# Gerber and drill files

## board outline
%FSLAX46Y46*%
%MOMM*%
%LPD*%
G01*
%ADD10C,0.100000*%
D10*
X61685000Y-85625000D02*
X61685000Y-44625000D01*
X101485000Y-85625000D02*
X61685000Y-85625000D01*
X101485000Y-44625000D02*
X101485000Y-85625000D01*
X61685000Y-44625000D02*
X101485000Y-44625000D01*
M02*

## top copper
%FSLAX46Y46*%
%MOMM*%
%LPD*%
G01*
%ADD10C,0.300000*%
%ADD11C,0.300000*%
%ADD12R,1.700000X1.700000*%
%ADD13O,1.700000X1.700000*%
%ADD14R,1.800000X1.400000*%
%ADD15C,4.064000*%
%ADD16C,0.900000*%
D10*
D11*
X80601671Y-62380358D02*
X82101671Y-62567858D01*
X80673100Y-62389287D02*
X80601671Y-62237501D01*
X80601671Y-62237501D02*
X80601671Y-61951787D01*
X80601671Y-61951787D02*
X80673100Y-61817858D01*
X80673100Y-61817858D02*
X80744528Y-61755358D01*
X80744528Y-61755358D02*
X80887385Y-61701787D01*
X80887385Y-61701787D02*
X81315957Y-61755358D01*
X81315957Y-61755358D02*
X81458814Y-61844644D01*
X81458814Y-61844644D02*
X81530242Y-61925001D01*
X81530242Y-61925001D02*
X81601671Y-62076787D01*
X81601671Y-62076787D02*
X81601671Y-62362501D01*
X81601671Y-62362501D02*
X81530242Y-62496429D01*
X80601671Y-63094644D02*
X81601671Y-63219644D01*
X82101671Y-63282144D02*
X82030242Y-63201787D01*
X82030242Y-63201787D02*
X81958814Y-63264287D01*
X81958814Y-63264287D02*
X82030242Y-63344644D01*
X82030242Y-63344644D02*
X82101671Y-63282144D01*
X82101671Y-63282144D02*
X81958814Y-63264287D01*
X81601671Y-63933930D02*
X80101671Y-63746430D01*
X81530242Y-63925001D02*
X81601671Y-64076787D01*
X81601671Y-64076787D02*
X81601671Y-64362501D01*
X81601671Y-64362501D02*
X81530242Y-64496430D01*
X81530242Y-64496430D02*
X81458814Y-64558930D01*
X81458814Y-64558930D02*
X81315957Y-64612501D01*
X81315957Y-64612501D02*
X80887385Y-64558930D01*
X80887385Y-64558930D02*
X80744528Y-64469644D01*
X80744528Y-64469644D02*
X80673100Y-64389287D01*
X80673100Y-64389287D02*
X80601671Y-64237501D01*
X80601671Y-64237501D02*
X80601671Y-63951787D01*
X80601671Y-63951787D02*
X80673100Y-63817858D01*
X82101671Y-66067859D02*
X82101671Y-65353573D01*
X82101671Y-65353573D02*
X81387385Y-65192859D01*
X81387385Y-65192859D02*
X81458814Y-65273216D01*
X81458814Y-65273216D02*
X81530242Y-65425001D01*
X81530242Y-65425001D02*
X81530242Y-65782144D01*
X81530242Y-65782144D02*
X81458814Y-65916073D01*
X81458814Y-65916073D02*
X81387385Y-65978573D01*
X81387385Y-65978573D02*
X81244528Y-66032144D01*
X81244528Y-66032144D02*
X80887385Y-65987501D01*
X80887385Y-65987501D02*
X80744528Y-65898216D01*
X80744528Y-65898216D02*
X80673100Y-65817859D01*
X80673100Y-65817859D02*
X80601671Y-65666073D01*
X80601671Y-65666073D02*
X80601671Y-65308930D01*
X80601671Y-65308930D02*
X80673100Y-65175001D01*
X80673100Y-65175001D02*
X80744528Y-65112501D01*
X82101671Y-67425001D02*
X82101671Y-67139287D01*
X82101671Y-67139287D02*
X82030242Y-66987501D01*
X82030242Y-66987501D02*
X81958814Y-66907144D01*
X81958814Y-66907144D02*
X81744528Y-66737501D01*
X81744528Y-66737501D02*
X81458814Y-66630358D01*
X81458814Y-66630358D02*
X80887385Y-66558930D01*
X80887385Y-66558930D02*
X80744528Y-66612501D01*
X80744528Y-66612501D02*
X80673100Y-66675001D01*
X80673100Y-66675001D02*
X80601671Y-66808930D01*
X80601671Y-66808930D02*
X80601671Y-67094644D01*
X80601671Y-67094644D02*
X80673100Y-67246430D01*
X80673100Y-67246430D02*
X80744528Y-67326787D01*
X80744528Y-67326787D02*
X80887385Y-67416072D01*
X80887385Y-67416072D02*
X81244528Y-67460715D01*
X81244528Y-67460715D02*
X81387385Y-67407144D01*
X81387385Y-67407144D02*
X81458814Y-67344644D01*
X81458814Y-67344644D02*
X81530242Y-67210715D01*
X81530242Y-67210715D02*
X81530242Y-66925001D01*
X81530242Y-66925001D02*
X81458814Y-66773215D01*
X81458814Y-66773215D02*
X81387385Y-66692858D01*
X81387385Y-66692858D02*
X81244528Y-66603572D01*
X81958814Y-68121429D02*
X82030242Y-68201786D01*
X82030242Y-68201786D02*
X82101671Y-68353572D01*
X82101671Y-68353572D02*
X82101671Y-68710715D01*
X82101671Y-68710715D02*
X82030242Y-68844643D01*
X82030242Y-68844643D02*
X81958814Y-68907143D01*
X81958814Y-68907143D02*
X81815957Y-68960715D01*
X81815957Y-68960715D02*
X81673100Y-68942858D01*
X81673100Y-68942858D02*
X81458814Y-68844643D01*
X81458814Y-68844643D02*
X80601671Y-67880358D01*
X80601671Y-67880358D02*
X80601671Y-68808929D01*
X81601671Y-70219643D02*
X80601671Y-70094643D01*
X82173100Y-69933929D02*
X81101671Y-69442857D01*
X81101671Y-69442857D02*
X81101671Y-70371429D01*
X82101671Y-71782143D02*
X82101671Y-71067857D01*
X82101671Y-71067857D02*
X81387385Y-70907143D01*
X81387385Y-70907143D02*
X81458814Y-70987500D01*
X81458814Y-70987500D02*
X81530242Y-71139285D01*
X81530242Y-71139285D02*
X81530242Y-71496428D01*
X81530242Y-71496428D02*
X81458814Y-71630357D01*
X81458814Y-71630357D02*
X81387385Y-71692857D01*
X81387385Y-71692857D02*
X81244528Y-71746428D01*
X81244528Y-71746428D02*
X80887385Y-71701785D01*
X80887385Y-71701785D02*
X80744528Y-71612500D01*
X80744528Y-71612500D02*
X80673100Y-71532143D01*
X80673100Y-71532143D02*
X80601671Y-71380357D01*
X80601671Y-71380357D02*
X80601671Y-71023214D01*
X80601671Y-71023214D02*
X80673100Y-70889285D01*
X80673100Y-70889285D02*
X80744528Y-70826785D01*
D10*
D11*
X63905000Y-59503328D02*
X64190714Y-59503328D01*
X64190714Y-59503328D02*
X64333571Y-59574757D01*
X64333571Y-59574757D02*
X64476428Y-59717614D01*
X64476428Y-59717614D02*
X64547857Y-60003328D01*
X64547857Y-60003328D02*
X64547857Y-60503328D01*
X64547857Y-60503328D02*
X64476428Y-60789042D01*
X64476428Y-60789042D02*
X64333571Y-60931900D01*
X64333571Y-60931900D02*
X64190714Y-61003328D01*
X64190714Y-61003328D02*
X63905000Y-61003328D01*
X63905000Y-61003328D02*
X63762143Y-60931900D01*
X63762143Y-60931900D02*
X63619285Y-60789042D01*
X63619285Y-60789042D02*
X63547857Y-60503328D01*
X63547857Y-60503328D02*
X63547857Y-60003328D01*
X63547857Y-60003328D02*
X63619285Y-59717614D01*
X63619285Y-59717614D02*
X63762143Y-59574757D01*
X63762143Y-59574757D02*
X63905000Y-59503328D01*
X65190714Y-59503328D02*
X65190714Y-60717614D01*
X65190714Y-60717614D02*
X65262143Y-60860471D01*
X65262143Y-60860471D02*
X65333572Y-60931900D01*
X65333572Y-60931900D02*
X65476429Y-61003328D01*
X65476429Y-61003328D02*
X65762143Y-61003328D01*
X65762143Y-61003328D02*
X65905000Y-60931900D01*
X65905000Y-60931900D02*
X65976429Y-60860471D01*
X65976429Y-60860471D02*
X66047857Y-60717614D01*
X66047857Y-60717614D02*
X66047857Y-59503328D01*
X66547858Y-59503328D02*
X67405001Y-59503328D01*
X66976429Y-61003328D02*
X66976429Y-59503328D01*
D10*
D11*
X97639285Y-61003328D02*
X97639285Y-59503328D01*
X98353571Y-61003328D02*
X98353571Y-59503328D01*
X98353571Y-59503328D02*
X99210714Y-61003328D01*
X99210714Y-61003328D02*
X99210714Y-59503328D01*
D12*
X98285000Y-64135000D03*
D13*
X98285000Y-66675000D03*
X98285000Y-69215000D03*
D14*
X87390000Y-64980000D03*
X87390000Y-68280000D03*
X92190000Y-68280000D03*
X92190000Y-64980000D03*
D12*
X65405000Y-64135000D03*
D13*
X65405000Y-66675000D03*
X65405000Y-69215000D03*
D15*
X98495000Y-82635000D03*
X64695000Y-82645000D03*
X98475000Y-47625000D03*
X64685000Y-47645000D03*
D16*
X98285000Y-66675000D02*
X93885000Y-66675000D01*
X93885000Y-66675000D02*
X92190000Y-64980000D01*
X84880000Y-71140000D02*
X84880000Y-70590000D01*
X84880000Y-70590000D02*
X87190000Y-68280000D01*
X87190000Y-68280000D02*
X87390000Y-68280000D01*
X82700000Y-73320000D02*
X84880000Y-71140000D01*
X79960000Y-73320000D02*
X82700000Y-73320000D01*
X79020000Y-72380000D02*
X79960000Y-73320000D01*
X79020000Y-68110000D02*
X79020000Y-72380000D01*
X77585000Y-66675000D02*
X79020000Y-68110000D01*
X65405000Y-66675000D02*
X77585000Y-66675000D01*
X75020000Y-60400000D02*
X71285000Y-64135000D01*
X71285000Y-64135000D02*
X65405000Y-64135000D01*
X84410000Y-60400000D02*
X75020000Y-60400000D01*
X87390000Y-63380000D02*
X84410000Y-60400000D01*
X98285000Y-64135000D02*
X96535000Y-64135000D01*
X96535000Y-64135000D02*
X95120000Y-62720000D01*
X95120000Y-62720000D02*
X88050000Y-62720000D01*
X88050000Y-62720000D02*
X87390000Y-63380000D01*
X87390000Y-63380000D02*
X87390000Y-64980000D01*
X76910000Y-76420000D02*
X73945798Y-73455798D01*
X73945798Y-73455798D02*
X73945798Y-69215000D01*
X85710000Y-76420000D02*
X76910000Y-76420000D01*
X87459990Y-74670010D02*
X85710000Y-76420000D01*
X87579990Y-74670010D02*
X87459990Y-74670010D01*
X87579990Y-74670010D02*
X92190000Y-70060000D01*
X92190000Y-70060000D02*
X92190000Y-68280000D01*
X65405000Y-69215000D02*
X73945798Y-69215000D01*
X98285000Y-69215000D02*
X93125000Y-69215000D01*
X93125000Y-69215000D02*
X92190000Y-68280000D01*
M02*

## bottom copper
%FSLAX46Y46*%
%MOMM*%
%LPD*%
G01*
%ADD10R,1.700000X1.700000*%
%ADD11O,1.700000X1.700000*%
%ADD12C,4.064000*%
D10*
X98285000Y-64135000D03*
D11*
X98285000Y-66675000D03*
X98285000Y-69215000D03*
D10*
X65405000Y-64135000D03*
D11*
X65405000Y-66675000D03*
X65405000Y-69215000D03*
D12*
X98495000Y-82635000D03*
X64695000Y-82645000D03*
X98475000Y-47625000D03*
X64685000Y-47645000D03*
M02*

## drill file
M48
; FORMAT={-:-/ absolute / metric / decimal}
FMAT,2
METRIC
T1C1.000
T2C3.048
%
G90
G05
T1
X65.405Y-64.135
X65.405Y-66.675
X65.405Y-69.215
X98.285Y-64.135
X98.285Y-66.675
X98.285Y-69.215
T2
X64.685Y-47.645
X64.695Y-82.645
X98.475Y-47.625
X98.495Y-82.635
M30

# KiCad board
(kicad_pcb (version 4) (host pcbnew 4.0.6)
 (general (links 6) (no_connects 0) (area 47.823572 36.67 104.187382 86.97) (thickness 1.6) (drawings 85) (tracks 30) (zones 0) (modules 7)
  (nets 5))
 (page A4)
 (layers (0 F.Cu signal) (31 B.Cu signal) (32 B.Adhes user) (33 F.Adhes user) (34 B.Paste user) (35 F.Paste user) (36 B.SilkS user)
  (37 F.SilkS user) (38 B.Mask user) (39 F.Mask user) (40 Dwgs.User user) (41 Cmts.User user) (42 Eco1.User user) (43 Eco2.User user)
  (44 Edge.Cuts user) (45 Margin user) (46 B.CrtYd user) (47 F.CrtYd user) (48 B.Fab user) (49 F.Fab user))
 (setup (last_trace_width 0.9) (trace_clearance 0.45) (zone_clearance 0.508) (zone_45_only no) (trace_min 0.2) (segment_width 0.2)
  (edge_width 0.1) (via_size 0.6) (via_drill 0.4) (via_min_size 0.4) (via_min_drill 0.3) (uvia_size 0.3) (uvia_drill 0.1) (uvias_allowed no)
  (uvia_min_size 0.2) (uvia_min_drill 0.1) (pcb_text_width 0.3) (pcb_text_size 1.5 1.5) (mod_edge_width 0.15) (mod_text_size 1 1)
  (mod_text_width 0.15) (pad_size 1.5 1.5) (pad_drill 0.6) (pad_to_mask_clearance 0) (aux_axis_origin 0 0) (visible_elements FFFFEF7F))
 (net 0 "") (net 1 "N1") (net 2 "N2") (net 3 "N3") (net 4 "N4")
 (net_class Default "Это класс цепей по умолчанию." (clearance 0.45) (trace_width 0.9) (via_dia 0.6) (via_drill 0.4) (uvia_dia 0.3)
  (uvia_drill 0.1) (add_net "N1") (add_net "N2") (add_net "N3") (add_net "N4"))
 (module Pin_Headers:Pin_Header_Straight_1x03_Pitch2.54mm (layer F.Cu) (at 98.285 64.135)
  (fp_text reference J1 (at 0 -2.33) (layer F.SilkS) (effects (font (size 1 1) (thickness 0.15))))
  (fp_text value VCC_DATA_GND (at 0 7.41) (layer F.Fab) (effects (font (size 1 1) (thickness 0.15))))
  (pad 1 thru_hole rect (at 0 0) (size 1.7 1.7) (drill 1) (layers *.Cu *.Mask) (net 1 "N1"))
  (pad 2 thru_hole oval (at 0 2.54) (size 1.7 1.7) (drill 1) (layers *.Cu *.Mask) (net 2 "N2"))
  (pad 3 thru_hole oval (at 0 5.08) (size 1.7 1.7) (drill 1) (layers *.Cu *.Mask) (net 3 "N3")))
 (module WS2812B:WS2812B (layer F.Cu) (at 89.79 66.63 90)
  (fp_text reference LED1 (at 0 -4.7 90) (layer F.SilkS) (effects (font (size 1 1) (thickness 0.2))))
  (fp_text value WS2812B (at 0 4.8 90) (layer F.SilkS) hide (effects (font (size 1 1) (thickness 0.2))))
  (pad 1 smd rect (at 1.65 -2.4 90) (size 1.4 1.8) (layers F.Cu F.Paste F.Mask) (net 1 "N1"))
  (pad 2 smd rect (at -1.65 -2.4 90) (size 1.4 1.8) (layers F.Cu F.Paste F.Mask) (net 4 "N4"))
  (pad 3 smd rect (at -1.65 2.4 90) (size 1.4 1.8) (layers F.Cu F.Paste F.Mask) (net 3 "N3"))
  (pad 4 smd rect (at 1.65 2.4 90) (size 1.4 1.8) (layers F.Cu F.Paste F.Mask) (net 2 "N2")))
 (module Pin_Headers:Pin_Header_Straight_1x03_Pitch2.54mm (layer F.Cu) (at 65.405 64.135)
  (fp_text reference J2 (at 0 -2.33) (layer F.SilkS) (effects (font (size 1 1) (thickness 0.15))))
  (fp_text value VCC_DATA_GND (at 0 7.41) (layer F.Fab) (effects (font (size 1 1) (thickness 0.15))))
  (pad 1 thru_hole rect (at 0 0) (size 1.7 1.7) (drill 1) (layers *.Cu *.Mask) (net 1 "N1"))
  (pad 2 thru_hole oval (at 0 2.54) (size 1.7 1.7) (drill 1) (layers *.Cu *.Mask) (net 4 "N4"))
  (pad 3 thru_hole oval (at 0 5.08) (size 1.7 1.7) (drill 1) (layers *.Cu *.Mask) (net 3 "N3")))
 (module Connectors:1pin (layer F.Cu) (at 98.495 82.635)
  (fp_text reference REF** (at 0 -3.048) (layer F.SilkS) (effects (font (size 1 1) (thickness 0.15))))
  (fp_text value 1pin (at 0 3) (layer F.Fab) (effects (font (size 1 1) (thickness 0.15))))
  (pad 1 thru_hole circle (at 0 0) (size 4.064 4.064) (drill 3.048) (layers *.Cu *.Mask)))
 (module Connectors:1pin (layer F.Cu) (at 64.695 82.645)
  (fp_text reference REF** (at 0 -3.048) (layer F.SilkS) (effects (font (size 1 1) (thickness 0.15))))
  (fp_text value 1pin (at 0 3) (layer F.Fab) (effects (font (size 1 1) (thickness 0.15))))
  (pad 1 thru_hole circle (at 0 0) (size 4.064 4.064) (drill 3.048) (layers *.Cu *.Mask)))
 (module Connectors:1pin (layer F.Cu) (at 98.475 47.625)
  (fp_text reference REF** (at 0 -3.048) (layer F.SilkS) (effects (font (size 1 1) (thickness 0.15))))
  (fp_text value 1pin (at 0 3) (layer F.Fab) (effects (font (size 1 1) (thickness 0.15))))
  (pad 1 thru_hole circle (at 0 0) (size 4.064 4.064) (drill 3.048) (layers *.Cu *.Mask)))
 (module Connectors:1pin (layer F.Cu) (at 64.685 47.645)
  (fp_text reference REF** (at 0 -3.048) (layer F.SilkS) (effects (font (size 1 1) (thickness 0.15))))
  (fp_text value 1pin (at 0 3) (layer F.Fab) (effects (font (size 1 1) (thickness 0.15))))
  (pad 1 thru_hole circle (at 0 0) (size 4.064 4.064) (drill 3.048) (layers *.Cu *.Mask)))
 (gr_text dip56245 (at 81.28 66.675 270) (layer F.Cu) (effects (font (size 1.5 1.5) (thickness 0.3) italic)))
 (gr_line (start 61.685 85.625) (end 61.685 44.625) (layer Edge.Cuts) (width 0.1))
 (gr_line (start 101.485 85.625) (end 61.685 85.625) (layer Edge.Cuts) (width 0.1))
 (gr_line (start 101.485 44.625) (end 101.485 85.625) (layer Edge.Cuts) (width 0.1))
 (gr_line (start 61.685 44.625) (end 101.485 44.625) (layer Edge.Cuts) (width 0.1))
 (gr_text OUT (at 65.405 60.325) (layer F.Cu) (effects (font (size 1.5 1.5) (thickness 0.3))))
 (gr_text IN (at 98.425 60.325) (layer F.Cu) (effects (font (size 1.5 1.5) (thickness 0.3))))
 (segment (start 98.285 66.675) (end 93.885 66.675) (width 0.9) (layer F.Cu) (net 2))
 (segment (start 93.885 66.675) (end 92.19 64.98) (width 0.9) (layer F.Cu) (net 2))
 (segment (start 84.88 71.14) (end 84.88 70.59) (width 0.9) (layer F.Cu) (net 4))
 (segment (start 84.88 70.59) (end 87.19 68.28) (width 0.9) (layer F.Cu) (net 4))
 (segment (start 87.19 68.28) (end 87.39 68.28) (width 0.9) (layer F.Cu) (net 4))
 (segment (start 82.7 73.32) (end 84.88 71.14) (width 0.9) (layer F.Cu) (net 4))
 (segment (start 79.96 73.32) (end 82.7 73.32) (width 0.9) (layer F.Cu) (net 4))
 (segment (start 79.02 72.38) (end 79.96 73.32) (width 0.9) (layer F.Cu) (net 4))
 (segment (start 79.02 68.11) (end 79.02 72.38) (width 0.9) (layer F.Cu) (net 4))
 (segment (start 77.585 66.675) (end 79.02 68.11) (width 0.9) (layer F.Cu) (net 4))
 (segment (start 65.405 66.675) (end 77.585 66.675) (width 0.9) (layer F.Cu) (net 4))
 (segment (start 75.02 60.4) (end 71.285 64.135) (width 0.9) (layer F.Cu) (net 1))
 (segment (start 71.285 64.135) (end 65.405 64.135) (width 0.9) (layer F.Cu) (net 1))
 (segment (start 84.41 60.4) (end 75.02 60.4) (width 0.9) (layer F.Cu) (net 1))
 (segment (start 87.39 63.38) (end 84.41 60.4) (width 0.9) (layer F.Cu) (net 1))
 (segment (start 98.285 64.135) (end 96.535 64.135) (width 0.9) (layer F.Cu) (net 1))
 (segment (start 96.535 64.135) (end 95.12 62.72) (width 0.9) (layer F.Cu) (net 1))
 (segment (start 95.12 62.72) (end 88.05 62.72) (width 0.9) (layer F.Cu) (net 1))
 (segment (start 88.05 62.72) (end 87.39 63.38) (width 0.9) (layer F.Cu) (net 1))
 (segment (start 87.39 63.38) (end 87.39 64.98) (width 0.9) (layer F.Cu) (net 1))
 (segment (start 76.91 76.42) (end 73.945798 73.455798) (width 0.9) (layer F.Cu) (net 3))
 (segment (start 73.945798 73.455798) (end 73.945798 69.215) (width 0.9) (layer F.Cu) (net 3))
 (segment (start 85.71 76.42) (end 76.91 76.42) (width 0.9) (layer F.Cu) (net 3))
 (segment (start 87.45999 74.67001) (end 85.71 76.42) (width 0.9) (layer F.Cu) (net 3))
 (segment (start 87.57999 74.67001) (end 87.45999 74.67001) (width 0.9) (layer F.Cu) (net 3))
 (segment (start 87.57999 74.67001) (end 92.19 70.06) (width 0.9) (layer F.Cu) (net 3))
 (segment (start 92.19 70.06) (end 92.19 68.28) (width 0.9) (layer F.Cu) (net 3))
 (segment (start 65.405 69.215) (end 73.945798 69.215) (width 0.9) (layer F.Cu) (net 3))
 (segment (start 98.285 69.215) (end 93.125 69.215) (width 0.9) (layer F.Cu) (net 3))
 (segment (start 93.125 69.215) (end 92.19 68.28) (width 0.9) (layer F.Cu) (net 3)))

